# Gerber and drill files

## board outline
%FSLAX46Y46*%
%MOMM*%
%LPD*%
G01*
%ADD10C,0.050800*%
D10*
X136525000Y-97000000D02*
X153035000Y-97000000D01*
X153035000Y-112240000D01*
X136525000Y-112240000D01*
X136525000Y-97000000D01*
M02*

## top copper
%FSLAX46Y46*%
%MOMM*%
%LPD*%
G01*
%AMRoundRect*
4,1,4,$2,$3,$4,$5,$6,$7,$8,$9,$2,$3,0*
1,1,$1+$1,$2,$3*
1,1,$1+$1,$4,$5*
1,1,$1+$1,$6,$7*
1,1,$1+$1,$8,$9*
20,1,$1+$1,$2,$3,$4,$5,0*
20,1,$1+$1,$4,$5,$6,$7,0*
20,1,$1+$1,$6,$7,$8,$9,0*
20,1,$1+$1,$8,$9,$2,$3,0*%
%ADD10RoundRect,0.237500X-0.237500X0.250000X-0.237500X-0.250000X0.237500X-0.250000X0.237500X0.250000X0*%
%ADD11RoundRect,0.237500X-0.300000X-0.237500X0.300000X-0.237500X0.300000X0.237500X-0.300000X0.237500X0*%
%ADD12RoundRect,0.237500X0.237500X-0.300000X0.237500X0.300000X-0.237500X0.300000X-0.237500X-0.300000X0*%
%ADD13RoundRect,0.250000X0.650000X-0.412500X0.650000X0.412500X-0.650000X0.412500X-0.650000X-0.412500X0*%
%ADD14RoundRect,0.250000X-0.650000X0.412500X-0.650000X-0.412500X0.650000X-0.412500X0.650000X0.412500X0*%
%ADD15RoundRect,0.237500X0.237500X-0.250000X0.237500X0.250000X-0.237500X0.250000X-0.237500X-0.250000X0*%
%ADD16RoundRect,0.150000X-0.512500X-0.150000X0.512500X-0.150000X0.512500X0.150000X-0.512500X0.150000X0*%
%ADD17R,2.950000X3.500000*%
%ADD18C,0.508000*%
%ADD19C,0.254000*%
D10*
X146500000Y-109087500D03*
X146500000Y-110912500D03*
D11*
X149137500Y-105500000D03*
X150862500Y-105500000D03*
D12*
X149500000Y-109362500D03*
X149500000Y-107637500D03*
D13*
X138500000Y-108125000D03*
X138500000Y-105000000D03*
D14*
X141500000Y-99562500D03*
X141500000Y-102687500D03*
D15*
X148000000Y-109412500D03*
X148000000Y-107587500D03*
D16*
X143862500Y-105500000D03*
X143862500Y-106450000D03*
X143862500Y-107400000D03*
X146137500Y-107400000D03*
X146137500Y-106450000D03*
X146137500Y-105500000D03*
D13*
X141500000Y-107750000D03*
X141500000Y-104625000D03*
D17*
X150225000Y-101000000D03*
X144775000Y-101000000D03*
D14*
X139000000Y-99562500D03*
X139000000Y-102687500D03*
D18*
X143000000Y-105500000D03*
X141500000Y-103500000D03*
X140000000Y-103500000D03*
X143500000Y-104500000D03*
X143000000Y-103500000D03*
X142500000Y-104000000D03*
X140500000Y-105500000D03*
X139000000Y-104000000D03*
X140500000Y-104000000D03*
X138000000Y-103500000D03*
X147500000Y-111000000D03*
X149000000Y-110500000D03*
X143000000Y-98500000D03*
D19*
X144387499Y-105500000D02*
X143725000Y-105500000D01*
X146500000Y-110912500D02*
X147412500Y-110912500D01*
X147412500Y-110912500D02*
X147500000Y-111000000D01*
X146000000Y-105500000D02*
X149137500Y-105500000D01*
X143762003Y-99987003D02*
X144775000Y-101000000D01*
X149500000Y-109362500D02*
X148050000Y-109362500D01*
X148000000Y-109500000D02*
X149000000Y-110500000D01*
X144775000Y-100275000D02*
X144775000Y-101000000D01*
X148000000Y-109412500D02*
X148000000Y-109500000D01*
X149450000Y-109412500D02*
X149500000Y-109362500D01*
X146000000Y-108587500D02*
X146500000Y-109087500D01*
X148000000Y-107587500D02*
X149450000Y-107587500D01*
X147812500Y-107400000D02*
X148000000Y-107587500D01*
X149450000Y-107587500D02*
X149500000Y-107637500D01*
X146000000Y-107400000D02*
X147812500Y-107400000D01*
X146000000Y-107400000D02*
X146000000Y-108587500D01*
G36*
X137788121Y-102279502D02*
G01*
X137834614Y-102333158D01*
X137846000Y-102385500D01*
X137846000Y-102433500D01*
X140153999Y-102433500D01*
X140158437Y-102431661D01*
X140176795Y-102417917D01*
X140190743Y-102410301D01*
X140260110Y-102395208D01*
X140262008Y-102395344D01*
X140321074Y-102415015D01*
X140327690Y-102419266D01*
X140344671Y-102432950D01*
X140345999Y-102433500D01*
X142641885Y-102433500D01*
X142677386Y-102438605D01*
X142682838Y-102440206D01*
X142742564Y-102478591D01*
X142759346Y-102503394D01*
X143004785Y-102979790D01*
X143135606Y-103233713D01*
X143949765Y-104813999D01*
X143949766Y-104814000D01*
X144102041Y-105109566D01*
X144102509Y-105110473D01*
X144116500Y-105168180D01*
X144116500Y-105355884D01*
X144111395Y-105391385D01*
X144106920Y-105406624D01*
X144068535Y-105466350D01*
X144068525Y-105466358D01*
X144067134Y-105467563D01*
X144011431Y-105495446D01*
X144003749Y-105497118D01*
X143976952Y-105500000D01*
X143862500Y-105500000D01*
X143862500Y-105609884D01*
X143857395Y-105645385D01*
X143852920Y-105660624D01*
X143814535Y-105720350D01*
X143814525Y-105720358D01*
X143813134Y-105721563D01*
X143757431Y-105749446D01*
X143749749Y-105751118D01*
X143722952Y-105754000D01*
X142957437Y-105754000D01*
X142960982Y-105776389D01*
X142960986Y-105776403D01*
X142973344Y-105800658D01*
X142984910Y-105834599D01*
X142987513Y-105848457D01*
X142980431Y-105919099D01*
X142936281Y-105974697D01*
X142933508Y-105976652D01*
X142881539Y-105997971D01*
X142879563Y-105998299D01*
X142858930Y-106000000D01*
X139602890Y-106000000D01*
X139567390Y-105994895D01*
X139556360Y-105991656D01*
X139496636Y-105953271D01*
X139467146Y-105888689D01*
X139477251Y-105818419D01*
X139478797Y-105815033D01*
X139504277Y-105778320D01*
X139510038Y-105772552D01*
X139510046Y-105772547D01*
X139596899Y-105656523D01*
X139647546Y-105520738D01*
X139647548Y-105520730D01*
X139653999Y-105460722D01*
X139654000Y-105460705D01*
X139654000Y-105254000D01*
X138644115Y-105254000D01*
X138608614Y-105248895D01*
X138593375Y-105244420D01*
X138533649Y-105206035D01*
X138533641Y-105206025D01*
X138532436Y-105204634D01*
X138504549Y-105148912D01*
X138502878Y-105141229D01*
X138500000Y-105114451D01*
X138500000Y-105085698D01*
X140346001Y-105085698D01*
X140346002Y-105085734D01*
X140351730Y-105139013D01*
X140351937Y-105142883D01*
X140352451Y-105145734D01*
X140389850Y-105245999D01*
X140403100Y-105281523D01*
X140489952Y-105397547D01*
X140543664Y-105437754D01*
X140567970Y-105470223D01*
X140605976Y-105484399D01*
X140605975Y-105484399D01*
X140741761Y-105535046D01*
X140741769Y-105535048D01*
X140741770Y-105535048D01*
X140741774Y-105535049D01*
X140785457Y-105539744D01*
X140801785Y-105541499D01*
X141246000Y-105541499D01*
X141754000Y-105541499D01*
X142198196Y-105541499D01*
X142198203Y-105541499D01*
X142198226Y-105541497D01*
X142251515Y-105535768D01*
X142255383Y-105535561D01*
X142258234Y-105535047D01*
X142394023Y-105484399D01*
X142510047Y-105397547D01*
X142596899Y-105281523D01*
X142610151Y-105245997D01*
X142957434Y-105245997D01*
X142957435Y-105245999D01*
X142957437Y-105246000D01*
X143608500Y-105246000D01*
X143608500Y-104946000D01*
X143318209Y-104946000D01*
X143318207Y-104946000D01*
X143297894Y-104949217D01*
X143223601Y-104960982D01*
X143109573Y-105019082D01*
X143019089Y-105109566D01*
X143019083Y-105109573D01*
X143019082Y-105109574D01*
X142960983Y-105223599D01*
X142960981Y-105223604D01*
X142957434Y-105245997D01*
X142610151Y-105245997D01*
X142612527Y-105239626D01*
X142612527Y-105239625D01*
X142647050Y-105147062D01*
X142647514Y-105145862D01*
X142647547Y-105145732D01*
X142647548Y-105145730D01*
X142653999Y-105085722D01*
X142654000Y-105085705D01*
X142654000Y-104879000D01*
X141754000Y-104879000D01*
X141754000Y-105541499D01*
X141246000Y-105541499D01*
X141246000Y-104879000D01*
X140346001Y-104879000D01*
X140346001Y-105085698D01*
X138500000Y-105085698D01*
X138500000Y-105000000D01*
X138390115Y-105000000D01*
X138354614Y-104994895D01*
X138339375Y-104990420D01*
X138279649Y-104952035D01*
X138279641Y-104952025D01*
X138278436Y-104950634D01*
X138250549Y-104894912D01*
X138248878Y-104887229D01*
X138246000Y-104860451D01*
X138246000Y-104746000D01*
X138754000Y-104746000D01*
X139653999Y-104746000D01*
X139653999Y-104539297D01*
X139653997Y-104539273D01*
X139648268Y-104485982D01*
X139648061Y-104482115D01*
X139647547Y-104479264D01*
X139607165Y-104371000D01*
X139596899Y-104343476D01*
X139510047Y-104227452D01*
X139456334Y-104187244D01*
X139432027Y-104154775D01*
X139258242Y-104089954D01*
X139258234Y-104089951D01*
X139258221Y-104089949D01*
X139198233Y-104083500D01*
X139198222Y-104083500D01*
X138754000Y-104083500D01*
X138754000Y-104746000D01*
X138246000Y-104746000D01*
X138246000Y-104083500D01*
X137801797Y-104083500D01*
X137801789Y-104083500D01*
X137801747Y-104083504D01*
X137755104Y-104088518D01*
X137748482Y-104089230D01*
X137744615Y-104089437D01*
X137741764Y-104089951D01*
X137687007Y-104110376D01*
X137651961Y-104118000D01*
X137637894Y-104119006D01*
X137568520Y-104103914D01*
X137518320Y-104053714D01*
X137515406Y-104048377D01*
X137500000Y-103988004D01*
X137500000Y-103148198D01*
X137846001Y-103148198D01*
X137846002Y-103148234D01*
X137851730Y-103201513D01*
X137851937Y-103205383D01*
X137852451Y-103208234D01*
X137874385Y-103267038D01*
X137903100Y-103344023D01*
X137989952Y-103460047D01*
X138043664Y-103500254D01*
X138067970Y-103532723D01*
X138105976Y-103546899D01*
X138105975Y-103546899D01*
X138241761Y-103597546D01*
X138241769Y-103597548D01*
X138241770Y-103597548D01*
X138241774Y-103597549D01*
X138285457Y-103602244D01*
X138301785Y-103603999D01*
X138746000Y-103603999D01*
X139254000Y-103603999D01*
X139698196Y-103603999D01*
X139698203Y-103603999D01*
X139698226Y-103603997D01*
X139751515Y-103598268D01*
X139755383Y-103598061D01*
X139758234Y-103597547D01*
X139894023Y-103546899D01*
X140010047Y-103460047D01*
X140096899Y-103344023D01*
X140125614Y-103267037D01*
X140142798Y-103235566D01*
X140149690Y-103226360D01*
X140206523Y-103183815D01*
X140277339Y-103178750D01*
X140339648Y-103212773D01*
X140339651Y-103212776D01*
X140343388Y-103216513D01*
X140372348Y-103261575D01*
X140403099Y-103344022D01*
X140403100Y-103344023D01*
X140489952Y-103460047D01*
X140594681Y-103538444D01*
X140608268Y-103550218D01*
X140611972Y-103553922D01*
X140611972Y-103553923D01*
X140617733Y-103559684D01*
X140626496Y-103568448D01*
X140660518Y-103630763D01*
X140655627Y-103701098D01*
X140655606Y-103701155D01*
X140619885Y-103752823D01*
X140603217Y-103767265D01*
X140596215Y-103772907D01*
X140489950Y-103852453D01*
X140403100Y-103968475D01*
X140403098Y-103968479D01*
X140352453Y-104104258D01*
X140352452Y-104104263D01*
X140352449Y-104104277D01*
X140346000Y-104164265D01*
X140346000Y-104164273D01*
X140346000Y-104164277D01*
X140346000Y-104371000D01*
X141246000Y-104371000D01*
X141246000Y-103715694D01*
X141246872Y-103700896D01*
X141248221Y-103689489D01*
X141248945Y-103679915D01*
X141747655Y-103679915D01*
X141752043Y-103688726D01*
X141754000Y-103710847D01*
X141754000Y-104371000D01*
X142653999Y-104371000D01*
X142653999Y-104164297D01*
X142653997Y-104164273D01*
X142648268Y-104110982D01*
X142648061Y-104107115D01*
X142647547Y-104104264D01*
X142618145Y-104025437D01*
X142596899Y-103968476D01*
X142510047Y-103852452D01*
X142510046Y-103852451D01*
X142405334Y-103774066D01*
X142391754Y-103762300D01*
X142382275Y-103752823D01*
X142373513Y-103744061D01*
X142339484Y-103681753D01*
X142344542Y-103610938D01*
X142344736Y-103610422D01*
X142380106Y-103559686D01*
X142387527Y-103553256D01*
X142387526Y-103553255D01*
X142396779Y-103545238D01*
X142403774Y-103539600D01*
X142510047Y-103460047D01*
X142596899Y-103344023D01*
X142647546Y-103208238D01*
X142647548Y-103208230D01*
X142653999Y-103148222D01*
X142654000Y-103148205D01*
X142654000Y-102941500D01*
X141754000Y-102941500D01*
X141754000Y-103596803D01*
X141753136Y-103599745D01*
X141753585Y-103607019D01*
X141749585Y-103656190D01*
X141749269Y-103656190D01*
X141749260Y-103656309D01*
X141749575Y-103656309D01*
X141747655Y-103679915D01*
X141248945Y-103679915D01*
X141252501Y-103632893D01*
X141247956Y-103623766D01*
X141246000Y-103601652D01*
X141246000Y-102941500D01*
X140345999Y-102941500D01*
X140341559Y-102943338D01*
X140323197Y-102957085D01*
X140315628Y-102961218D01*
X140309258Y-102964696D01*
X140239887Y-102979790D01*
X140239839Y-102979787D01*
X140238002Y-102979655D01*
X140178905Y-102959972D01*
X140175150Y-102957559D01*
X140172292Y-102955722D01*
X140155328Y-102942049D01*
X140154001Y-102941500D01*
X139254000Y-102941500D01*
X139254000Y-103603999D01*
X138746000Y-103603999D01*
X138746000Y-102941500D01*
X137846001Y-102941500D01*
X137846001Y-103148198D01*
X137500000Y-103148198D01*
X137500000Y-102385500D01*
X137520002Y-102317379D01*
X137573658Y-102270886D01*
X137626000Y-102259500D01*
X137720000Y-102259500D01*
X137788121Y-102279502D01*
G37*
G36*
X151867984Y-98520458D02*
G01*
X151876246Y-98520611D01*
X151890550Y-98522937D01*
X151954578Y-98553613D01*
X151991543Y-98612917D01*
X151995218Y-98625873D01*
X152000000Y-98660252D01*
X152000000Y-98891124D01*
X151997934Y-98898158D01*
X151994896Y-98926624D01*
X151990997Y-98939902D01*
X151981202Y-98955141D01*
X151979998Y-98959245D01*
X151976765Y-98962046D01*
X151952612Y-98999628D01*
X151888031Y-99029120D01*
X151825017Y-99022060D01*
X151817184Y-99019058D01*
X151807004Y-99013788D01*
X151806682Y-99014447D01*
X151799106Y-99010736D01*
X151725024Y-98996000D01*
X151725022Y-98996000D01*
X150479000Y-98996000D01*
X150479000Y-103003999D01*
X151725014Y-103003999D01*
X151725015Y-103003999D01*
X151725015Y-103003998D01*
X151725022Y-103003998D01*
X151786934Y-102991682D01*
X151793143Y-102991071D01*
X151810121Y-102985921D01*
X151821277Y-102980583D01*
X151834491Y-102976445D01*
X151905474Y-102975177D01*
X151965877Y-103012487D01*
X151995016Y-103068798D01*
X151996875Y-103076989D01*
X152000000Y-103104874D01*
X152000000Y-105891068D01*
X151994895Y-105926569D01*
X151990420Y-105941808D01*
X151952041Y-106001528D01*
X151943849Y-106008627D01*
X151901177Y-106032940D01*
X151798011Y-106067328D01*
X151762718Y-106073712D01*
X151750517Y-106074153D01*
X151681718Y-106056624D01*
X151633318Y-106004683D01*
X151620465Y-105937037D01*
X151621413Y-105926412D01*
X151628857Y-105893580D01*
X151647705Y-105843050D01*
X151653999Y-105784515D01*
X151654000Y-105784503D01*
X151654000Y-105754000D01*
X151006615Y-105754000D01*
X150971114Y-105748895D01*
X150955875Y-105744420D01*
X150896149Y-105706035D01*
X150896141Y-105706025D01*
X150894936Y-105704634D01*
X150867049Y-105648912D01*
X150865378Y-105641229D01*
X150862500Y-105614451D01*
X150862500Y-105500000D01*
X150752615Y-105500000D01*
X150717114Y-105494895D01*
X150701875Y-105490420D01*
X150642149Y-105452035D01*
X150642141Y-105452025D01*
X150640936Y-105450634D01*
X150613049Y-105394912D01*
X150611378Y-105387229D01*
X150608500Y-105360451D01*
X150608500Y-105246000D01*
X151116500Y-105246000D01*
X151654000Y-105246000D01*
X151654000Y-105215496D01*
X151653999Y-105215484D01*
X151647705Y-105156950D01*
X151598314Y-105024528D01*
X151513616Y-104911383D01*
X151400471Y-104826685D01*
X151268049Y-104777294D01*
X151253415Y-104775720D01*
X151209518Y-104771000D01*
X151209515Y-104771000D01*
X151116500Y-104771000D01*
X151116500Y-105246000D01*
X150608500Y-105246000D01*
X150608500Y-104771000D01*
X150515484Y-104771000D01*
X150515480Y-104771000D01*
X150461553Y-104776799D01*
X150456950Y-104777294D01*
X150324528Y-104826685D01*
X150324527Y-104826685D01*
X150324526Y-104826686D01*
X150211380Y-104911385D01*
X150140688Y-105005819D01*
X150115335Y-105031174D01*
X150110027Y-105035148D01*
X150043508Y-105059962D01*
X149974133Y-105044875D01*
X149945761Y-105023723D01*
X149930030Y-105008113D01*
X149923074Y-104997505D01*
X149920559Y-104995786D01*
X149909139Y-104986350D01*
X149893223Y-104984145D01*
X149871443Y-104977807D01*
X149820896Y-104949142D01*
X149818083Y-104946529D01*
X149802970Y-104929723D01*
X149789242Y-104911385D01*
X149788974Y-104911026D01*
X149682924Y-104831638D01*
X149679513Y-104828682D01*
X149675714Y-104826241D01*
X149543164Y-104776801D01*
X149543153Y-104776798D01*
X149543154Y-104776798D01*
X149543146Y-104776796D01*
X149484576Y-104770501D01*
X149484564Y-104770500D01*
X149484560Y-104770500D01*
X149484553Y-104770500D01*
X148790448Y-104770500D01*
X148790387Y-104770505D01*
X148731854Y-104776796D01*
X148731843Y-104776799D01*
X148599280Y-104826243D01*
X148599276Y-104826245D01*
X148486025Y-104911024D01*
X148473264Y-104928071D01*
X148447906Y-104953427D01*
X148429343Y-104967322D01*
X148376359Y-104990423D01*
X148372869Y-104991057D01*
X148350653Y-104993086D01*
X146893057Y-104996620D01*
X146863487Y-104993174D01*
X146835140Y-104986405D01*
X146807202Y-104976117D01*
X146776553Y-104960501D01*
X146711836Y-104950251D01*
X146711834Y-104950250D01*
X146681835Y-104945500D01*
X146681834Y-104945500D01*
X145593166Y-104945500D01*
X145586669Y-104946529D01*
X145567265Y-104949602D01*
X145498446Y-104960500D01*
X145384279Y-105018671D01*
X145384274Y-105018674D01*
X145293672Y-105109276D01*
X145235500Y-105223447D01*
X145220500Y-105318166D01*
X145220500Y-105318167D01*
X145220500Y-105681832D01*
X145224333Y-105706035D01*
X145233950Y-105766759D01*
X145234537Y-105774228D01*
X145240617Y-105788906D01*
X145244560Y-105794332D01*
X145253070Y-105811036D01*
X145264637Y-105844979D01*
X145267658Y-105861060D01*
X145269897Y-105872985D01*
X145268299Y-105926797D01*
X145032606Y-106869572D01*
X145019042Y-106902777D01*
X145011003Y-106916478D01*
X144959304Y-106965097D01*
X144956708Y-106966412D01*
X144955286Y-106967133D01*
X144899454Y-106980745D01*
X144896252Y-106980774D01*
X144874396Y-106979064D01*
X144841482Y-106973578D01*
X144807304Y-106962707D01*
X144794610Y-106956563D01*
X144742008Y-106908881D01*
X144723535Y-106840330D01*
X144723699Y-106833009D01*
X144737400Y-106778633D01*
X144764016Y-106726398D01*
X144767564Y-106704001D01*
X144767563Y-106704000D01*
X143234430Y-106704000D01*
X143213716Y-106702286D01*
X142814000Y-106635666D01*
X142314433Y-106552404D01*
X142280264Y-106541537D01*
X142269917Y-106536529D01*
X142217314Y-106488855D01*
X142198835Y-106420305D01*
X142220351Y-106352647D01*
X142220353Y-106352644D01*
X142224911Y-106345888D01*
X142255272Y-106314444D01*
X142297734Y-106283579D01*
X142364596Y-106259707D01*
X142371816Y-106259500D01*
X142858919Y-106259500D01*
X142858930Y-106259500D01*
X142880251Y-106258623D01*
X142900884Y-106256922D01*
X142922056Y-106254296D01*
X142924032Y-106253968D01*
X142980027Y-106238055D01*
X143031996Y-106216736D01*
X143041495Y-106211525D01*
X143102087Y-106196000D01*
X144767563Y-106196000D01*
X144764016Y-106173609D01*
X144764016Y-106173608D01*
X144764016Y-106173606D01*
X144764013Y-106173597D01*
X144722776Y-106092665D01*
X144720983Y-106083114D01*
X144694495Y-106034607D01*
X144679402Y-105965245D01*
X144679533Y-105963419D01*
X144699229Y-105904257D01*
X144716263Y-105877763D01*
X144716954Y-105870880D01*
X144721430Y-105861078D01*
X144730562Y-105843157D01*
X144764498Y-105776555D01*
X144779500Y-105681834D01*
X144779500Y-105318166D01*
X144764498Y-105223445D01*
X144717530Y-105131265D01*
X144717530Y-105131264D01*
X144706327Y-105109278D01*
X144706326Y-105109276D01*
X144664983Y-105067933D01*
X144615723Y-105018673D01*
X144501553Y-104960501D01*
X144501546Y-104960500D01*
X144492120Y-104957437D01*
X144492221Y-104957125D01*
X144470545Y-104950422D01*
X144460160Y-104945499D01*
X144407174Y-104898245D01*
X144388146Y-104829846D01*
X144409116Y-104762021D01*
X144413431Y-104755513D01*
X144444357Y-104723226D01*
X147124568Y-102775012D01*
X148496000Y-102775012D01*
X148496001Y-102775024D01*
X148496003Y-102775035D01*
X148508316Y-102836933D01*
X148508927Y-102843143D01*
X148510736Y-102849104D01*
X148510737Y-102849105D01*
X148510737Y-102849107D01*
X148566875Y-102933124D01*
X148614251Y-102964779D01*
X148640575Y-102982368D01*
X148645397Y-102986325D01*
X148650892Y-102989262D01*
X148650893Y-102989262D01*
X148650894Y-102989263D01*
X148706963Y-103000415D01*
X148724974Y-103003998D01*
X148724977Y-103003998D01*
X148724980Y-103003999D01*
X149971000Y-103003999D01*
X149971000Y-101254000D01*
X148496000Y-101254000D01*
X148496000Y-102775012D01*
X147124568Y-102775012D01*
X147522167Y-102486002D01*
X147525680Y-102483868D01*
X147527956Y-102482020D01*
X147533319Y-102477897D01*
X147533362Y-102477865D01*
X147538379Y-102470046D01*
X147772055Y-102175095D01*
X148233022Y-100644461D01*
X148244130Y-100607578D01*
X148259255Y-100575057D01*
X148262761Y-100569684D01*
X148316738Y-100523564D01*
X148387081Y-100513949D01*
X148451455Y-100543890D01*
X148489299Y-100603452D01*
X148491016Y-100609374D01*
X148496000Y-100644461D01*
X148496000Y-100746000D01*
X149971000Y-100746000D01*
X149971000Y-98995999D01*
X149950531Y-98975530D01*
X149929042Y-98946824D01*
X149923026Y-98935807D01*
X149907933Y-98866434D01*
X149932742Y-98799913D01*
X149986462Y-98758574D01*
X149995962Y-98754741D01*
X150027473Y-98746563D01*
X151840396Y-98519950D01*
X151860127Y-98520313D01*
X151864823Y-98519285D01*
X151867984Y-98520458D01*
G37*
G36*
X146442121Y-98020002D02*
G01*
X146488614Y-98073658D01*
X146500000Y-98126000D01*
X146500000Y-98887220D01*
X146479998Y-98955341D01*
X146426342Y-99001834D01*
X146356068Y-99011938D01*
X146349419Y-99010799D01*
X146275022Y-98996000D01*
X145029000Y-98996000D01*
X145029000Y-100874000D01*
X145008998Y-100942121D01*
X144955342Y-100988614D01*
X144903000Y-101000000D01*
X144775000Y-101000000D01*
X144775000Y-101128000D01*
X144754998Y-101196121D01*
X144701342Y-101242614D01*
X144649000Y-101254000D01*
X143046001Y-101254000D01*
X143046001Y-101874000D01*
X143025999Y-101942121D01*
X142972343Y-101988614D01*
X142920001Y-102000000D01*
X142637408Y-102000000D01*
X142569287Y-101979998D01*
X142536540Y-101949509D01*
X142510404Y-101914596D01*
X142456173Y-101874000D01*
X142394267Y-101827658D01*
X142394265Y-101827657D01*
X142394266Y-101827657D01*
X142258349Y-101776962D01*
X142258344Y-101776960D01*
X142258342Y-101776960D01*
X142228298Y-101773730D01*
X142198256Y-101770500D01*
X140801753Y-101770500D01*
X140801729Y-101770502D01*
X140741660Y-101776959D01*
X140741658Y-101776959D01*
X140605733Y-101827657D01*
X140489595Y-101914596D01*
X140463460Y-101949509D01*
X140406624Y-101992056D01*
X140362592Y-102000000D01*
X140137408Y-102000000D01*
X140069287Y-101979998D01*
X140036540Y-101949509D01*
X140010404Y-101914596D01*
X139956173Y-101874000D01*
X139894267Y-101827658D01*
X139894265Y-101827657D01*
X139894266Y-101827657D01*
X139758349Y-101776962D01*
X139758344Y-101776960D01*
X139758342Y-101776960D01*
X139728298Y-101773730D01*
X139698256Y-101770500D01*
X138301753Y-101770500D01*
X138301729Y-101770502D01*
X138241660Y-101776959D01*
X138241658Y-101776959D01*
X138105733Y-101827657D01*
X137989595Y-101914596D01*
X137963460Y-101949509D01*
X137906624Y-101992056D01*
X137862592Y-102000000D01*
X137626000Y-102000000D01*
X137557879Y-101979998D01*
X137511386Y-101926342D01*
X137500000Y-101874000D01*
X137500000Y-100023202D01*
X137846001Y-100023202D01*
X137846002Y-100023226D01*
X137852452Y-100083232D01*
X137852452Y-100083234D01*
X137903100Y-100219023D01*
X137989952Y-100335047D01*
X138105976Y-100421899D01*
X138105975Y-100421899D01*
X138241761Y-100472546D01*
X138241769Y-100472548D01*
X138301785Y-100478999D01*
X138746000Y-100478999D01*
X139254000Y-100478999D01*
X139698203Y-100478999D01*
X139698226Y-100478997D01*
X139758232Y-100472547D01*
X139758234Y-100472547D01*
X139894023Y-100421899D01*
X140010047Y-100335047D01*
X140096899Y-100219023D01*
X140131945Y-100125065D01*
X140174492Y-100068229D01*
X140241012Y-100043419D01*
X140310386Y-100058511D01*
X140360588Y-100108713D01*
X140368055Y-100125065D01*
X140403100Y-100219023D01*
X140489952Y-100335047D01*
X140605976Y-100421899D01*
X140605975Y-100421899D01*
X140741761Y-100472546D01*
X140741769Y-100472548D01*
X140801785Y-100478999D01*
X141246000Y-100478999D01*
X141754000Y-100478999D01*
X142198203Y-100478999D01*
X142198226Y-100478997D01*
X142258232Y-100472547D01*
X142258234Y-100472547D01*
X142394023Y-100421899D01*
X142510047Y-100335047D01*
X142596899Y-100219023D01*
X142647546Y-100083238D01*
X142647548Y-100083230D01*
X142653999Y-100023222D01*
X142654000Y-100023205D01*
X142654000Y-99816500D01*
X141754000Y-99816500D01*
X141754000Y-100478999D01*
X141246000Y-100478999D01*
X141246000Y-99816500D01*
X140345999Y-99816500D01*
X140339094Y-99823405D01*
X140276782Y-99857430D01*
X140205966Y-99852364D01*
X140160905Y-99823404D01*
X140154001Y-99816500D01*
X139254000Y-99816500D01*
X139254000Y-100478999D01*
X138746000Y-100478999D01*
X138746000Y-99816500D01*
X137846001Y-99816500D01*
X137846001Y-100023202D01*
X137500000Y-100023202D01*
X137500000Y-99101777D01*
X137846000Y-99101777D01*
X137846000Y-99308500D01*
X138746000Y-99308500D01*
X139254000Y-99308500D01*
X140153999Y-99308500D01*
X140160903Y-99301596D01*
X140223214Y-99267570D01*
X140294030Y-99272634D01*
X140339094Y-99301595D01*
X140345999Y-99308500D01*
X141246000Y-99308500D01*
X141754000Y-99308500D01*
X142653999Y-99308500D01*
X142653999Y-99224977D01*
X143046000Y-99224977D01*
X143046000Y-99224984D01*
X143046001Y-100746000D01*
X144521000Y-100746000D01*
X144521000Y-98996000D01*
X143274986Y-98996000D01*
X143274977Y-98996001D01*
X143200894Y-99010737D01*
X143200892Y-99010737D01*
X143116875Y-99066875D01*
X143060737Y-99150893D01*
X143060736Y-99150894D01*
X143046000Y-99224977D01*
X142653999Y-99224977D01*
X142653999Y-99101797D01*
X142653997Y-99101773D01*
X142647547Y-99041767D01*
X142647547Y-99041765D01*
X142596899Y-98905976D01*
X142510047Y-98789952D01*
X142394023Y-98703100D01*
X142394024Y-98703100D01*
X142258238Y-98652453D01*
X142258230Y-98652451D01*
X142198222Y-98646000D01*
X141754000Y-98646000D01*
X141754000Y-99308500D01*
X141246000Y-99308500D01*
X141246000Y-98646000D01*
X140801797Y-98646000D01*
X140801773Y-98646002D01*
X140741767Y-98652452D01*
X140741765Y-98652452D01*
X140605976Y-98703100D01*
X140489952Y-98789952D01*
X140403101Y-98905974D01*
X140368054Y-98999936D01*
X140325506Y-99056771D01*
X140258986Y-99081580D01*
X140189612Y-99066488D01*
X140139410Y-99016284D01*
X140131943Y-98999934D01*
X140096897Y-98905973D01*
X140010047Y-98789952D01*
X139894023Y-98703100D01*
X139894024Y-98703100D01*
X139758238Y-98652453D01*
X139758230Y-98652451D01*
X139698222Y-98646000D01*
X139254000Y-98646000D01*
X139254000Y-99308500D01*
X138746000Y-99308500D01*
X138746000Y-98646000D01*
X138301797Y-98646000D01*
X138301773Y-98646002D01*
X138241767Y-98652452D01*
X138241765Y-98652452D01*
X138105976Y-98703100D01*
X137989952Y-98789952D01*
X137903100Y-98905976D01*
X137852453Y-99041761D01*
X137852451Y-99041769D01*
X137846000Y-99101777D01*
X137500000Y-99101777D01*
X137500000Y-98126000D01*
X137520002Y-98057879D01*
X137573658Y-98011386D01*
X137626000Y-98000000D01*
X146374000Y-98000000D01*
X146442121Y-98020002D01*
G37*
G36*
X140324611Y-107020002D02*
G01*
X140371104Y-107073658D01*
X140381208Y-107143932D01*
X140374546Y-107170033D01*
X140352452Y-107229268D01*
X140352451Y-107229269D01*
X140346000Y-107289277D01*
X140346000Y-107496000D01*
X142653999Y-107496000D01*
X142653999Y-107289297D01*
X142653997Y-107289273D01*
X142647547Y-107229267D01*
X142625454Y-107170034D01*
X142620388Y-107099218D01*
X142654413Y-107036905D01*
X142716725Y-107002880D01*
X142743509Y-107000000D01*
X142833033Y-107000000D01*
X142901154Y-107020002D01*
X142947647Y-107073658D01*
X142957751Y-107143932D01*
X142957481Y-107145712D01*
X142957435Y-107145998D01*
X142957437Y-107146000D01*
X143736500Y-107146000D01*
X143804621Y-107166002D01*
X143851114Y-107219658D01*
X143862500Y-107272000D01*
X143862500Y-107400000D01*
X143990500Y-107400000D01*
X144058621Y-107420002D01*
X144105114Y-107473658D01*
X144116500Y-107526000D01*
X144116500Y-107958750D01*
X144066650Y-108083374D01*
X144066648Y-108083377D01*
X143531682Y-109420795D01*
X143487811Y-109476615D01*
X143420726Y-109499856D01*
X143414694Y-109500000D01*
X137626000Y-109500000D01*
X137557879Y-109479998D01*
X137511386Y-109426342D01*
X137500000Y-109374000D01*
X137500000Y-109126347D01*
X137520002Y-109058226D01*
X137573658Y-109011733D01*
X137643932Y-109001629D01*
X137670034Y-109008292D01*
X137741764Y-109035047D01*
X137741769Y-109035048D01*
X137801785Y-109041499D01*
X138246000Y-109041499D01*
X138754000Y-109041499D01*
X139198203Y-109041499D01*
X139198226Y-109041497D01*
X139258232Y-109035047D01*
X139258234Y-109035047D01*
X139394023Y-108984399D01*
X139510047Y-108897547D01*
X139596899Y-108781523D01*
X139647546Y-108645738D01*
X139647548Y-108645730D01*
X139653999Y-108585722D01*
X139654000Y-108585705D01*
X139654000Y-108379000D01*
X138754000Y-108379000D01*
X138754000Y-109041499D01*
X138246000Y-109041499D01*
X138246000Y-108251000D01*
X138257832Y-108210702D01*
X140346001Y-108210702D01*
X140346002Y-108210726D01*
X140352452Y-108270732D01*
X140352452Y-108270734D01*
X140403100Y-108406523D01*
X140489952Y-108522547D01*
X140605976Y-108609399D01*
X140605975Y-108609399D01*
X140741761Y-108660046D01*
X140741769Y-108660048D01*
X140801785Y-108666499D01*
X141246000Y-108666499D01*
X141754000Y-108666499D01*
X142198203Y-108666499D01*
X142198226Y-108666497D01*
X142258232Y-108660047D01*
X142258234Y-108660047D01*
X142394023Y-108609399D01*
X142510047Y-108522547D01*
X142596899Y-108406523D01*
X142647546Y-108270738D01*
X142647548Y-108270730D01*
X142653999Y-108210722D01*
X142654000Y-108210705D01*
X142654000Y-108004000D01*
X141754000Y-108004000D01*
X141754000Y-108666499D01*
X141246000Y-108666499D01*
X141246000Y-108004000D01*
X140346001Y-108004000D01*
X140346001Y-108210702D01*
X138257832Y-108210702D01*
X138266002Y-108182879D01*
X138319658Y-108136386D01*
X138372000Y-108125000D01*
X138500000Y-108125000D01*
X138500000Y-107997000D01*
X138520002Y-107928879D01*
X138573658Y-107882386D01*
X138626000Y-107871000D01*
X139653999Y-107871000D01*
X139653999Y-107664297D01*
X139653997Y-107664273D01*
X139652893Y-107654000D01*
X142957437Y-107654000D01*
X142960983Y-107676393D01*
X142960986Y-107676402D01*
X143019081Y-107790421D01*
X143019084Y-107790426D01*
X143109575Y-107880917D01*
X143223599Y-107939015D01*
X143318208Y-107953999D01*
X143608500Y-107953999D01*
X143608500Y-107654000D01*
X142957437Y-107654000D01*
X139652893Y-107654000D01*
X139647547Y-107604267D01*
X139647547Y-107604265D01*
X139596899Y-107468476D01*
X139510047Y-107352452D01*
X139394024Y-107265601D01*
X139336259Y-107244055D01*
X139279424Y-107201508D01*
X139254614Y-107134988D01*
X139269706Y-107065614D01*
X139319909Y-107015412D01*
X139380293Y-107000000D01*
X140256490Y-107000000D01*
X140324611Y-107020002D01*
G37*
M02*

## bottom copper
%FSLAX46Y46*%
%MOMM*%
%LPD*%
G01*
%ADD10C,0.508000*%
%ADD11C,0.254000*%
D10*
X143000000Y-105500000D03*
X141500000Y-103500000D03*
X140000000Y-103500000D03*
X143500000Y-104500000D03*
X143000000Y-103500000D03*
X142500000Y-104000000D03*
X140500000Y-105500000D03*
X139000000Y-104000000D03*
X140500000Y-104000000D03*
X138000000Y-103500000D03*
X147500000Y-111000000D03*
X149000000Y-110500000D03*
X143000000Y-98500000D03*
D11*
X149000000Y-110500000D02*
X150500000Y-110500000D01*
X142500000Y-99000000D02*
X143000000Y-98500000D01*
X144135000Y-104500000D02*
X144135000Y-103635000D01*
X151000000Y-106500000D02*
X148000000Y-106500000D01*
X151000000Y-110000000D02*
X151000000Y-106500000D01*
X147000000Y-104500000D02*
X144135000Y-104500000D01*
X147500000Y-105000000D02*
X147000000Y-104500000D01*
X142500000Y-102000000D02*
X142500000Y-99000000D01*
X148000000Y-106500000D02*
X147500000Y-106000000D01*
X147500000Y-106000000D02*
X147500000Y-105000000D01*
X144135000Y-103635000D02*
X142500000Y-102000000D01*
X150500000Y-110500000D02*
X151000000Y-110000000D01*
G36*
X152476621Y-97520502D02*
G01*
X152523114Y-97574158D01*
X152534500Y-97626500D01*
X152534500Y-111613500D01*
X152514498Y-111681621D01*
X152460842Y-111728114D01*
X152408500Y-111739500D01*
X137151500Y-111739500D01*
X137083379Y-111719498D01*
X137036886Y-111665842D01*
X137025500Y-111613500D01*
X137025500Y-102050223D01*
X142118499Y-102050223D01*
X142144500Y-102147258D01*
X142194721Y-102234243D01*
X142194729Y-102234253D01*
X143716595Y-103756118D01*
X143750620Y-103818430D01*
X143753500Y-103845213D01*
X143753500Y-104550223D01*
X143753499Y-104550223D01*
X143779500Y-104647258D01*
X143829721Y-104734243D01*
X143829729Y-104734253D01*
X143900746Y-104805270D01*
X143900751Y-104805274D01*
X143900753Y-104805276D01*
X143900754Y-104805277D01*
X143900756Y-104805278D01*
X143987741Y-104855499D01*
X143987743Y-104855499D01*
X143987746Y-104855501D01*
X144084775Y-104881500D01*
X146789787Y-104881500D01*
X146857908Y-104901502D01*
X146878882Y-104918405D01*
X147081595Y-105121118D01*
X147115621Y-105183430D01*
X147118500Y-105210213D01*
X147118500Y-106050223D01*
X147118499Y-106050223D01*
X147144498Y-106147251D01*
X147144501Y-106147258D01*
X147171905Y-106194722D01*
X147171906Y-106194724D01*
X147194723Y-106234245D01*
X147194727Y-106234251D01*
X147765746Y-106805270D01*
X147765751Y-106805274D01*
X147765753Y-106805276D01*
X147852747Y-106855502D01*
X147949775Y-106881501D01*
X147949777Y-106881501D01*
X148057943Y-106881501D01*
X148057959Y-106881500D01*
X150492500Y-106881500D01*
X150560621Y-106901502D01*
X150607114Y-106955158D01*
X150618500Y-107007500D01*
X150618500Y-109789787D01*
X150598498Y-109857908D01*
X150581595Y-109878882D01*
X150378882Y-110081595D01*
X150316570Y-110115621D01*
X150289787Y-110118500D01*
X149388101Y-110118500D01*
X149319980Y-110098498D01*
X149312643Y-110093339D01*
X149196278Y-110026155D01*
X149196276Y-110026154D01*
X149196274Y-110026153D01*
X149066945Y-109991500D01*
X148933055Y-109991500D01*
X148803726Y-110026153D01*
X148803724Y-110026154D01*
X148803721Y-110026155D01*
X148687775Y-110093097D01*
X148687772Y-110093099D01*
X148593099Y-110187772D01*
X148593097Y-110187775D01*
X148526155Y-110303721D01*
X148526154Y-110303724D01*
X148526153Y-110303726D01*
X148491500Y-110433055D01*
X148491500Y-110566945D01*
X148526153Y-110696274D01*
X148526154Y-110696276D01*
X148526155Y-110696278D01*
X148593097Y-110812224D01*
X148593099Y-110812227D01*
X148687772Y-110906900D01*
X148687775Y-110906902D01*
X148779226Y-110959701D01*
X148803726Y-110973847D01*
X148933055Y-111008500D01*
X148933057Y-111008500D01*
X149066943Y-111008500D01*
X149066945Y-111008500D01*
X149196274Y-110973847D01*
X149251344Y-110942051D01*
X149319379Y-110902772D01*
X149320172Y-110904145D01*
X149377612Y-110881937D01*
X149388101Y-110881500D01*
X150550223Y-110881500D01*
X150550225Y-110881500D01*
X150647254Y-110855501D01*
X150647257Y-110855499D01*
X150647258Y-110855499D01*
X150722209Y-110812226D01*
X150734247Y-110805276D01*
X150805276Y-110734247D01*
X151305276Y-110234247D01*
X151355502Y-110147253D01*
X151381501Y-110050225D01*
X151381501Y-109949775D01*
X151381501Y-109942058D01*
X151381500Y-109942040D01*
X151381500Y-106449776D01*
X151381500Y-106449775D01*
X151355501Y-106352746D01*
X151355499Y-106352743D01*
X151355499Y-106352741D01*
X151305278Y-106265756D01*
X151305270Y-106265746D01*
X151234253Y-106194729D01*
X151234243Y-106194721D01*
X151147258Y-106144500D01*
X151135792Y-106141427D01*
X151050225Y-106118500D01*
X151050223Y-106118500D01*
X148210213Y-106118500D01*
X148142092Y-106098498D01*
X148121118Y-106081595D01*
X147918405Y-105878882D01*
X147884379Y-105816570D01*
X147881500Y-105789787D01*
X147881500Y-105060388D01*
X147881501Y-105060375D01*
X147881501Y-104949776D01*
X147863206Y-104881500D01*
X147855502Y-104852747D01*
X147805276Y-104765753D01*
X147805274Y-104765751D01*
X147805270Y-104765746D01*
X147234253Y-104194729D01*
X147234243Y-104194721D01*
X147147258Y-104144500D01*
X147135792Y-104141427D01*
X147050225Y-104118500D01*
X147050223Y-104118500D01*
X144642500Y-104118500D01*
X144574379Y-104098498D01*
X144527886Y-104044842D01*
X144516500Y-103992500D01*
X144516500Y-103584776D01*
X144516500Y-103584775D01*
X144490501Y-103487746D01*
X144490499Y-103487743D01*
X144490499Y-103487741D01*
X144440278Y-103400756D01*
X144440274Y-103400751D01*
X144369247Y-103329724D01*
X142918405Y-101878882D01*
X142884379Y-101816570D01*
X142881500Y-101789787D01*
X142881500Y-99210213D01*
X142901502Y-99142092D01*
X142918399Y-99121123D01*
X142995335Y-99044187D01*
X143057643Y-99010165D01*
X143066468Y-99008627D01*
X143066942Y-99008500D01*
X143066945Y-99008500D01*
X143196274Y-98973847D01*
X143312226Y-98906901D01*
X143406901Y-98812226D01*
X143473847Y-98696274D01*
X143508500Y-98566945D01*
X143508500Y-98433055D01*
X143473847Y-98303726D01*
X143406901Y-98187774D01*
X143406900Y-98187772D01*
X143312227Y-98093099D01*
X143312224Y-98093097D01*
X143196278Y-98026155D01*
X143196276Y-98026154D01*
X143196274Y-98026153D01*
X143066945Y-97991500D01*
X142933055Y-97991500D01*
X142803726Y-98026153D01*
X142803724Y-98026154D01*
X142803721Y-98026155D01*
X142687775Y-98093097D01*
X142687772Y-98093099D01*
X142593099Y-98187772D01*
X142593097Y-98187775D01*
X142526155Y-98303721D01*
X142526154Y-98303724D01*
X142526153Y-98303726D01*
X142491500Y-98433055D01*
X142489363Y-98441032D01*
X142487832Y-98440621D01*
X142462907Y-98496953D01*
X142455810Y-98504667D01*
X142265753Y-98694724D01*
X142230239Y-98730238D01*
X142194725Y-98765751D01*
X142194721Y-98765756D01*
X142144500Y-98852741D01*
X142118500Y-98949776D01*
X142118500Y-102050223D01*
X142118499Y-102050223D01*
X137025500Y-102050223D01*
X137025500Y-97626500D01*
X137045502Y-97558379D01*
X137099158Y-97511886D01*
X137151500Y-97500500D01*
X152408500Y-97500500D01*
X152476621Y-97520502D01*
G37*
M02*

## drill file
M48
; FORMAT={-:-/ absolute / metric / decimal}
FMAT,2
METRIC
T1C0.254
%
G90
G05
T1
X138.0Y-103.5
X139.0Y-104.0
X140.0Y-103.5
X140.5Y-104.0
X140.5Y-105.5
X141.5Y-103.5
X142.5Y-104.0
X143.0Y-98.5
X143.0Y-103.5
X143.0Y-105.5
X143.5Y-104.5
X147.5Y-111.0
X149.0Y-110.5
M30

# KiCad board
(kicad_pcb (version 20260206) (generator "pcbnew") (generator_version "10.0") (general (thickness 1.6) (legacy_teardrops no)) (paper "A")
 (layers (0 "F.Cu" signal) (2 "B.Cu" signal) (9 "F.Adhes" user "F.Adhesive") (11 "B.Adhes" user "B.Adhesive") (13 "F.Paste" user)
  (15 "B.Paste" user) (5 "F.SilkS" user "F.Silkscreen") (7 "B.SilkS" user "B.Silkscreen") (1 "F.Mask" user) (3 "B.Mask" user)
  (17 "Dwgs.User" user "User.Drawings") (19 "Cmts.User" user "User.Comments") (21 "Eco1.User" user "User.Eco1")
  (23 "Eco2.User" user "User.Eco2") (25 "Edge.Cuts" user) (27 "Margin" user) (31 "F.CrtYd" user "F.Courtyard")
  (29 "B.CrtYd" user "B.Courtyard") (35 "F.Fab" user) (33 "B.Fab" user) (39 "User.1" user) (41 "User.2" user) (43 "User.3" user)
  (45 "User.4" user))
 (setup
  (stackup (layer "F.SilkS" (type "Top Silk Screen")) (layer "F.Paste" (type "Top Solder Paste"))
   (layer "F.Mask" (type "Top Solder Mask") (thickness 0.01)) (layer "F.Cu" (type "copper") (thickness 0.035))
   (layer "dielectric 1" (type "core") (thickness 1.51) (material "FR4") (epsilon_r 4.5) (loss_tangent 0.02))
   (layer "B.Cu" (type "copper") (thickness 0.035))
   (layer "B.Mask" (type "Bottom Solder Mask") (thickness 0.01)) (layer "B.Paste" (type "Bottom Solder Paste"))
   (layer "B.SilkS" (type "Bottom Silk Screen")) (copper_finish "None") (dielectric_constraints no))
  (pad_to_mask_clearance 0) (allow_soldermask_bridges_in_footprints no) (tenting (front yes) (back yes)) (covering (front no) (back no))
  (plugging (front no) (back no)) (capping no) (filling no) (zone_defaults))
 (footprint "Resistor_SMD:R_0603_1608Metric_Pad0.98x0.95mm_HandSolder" (layer "F.Cu") (at 146.5 110 -90)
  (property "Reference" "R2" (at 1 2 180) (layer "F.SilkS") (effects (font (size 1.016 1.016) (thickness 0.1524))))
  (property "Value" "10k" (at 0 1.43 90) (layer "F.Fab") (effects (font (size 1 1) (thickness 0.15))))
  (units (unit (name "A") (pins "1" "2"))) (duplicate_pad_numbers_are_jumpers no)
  (pad "1" smd roundrect (at -0.9125 0 270) (size 0.975 0.95) (layers "F.Cu" "F.Mask" "F.Paste") (roundrect_rratio 0.25) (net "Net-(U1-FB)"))
  (pad "2" smd roundrect (at 0.9125 0 270) (size 0.975 0.95) (layers "F.Cu" "F.Mask" "F.Paste") (roundrect_rratio 0.25) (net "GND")))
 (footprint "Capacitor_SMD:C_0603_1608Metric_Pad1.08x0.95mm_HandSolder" (layer "F.Cu") (at 150 105.5)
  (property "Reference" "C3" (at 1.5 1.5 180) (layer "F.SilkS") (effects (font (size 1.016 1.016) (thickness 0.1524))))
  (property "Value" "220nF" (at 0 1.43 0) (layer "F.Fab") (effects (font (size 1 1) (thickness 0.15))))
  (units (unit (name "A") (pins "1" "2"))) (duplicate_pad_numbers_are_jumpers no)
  (pad "1" smd roundrect (at -0.8625 0) (size 1.075 0.95) (layers "F.Cu" "F.Mask" "F.Paste") (roundrect_rratio 0.25) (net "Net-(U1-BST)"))
  (pad "2" smd roundrect (at 0.8625 0) (size 1.075 0.95) (layers "F.Cu" "F.Mask" "F.Paste") (roundrect_rratio 0.25) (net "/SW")))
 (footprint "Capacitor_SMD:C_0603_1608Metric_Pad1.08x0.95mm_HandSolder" (layer "F.Cu") (at 149.5 108.5 90)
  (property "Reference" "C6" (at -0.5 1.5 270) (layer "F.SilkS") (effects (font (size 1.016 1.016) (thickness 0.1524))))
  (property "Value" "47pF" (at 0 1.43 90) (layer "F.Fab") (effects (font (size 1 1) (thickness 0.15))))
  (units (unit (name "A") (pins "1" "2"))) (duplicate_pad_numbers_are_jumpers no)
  (pad "1" smd roundrect (at -0.8625 0 90) (size 1.075 0.95) (layers "F.Cu" "F.Mask" "F.Paste") (roundrect_rratio 0.25) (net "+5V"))
  (pad "2" smd roundrect (at 0.8625 0 90) (size 1.075 0.95) (layers "F.Cu" "F.Mask" "F.Paste") (roundrect_rratio 0.25) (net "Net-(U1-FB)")))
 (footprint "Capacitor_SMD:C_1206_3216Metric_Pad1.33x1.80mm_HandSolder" (layer "F.Cu") (at 138.5 106.5625 90)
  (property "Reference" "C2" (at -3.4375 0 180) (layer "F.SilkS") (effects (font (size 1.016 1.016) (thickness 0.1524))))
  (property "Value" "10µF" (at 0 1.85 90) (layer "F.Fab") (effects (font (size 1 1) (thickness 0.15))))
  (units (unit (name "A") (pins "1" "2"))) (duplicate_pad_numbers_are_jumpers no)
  (pad "1" smd roundrect (at -1.5625 0 90) (size 1.325 1.8) (layers "F.Cu" "F.Mask" "F.Paste") (roundrect_rratio 0.188679) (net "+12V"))
  (pad "2" smd roundrect (at 1.5625 0 90) (size 1.325 1.8) (layers "F.Cu" "F.Mask" "F.Paste") (roundrect_rratio 0.188679) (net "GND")))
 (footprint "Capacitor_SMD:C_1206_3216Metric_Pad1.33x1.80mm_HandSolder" (layer "F.Cu") (at 141.5 101.125 -90)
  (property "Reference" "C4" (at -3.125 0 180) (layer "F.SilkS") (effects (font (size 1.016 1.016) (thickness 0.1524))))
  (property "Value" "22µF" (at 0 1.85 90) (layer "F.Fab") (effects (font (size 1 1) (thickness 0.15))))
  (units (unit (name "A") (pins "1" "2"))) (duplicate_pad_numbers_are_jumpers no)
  (pad "1" smd roundrect (at -1.5625 0 270) (size 1.325 1.8) (layers "F.Cu" "F.Mask" "F.Paste") (roundrect_rratio 0.188679) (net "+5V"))
  (pad "2" smd roundrect (at 1.5625 0 270) (size 1.325 1.8) (layers "F.Cu" "F.Mask" "F.Paste") (roundrect_rratio 0.188679) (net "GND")))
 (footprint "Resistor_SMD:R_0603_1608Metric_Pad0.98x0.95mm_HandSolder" (layer "F.Cu") (at 148 108.5 90)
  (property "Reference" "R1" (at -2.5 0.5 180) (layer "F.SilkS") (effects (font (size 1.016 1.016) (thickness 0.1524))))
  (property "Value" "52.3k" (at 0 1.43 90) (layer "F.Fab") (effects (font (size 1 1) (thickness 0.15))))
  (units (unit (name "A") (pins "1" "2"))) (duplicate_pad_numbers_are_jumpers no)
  (pad "1" smd roundrect (at -0.9125 0 90) (size 0.975 0.95) (layers "F.Cu" "F.Mask" "F.Paste") (roundrect_rratio 0.25) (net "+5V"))
  (pad "2" smd roundrect (at 0.9125 0 90) (size 0.975 0.95) (layers "F.Cu" "F.Mask" "F.Paste") (roundrect_rratio 0.25) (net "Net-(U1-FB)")))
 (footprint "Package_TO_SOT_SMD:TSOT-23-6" (layer "F.Cu") (at 145 106.45)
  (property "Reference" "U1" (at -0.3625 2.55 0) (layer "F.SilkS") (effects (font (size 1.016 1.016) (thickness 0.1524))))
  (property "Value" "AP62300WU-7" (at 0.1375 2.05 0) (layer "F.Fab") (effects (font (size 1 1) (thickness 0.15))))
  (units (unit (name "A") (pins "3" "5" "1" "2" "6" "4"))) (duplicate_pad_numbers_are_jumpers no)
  (pad "1" smd roundrect (at -1.1375 -0.95) (size 1.325 0.6) (layers "F.Cu" "F.Mask" "F.Paste") (roundrect_rratio 0.25) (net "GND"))
  (pad "2" smd roundrect (at -1.1375 0) (size 1.325 0.6) (layers "F.Cu" "F.Mask" "F.Paste") (roundrect_rratio 0.25) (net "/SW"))
  (pad "3" smd roundrect (at -1.1375 0.95) (size 1.325 0.6) (layers "F.Cu" "F.Mask" "F.Paste") (roundrect_rratio 0.25) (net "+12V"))
  (pad "4" smd roundrect (at 1.1375 0.95) (size 1.325 0.6) (layers "F.Cu" "F.Mask" "F.Paste") (roundrect_rratio 0.25) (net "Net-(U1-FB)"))
  (pad "5" smd roundrect (at 1.1375 0) (size 1.325 0.6) (layers "F.Cu" "F.Mask" "F.Paste") (roundrect_rratio 0.25)
   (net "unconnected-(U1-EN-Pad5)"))
  (pad "6" smd roundrect (at 1.1375 -0.95) (size 1.325 0.6) (layers "F.Cu" "F.Mask" "F.Paste") (roundrect_rratio 0.25) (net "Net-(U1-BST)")))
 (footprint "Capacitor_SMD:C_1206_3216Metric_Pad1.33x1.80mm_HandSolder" (layer "F.Cu") (at 141.5 106.1875 90)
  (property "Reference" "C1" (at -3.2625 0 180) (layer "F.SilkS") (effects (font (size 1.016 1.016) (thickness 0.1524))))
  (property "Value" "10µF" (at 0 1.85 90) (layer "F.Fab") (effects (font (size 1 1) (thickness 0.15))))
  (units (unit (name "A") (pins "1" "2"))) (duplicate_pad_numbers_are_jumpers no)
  (pad "1" smd roundrect (at -1.5625 0 90) (size 1.325 1.8) (layers "F.Cu" "F.Mask" "F.Paste") (roundrect_rratio 0.188679) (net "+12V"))
  (pad "2" smd roundrect (at 1.5625 0 90) (size 1.325 1.8) (layers "F.Cu" "F.Mask" "F.Paste") (roundrect_rratio 0.188679) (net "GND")))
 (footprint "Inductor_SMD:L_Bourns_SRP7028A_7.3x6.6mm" (layer "F.Cu") (at 147.5 101 180)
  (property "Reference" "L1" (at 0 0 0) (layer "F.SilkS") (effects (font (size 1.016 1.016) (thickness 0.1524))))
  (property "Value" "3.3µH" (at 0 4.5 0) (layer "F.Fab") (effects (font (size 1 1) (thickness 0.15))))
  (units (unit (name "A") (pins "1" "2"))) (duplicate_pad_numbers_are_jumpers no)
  (pad "1" smd rect (at -2.725 0 180) (size 2.95 3.5) (layers "F.Cu" "F.Mask" "F.Paste") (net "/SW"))
  (pad "2" smd rect (at 2.725 0 180) (size 2.95 3.5) (layers "F.Cu" "F.Mask" "F.Paste") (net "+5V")))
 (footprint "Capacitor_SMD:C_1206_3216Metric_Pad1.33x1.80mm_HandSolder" (layer "F.Cu") (at 139 101.125 -90)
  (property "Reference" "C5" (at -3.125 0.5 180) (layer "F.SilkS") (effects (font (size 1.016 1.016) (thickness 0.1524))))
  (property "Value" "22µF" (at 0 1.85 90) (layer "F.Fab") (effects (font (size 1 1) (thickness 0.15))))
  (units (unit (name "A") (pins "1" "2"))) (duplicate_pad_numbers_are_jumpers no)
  (pad "1" smd roundrect (at -1.5625 0 270) (size 1.325 1.8) (layers "F.Cu" "F.Mask" "F.Paste") (roundrect_rratio 0.188679) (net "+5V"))
  (pad "2" smd roundrect (at 1.5625 0 270) (size 1.325 1.8) (layers "F.Cu" "F.Mask" "F.Paste") (roundrect_rratio 0.188679) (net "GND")))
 (gr_rect (start 136.525 97) (end 153.035 112.24) (stroke (width 0.0508) (type solid)) (fill no) (layer "Edge.Cuts"))
 (segment (start 144.387499 105.5) (end 143.725 105.5) (width 0.254) (layer "F.Cu") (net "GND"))
 (segment (start 146.5 110.9125) (end 147.4125 110.9125) (width 0.254) (layer "F.Cu") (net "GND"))
 (segment (start 147.4125 110.9125) (end 147.5 111) (width 0.254) (layer "F.Cu") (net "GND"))
 (via (at 143 105.5) (size 0.508) (drill 0.254) (layers "F.Cu" "B.Cu") (free yes) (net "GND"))
 (via (at 141.5 103.5) (size 0.508) (drill 0.254) (layers "F.Cu" "B.Cu") (free yes) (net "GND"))
 (via (at 140 103.5) (size 0.508) (drill 0.254) (layers "F.Cu" "B.Cu") (free yes) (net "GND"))
 (via (at 143.5 104.5) (size 0.508) (drill 0.254) (layers "F.Cu" "B.Cu") (free yes) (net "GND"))
 (via (at 143 103.5) (size 0.508) (drill 0.254) (layers "F.Cu" "B.Cu") (free yes) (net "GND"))
 (via (at 142.5 104) (size 0.508) (drill 0.254) (layers "F.Cu" "B.Cu") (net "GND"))
 (via (at 140.5 105.5) (size 0.508) (drill 0.254) (layers "F.Cu" "B.Cu") (free yes) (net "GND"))
 (via (at 139 104) (size 0.508) (drill 0.254) (layers "F.Cu" "B.Cu") (free yes) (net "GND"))
 (via (at 140.5 104) (size 0.508) (drill 0.254) (layers "F.Cu" "B.Cu") (free yes) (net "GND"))
 (via (at 138 103.5) (size 0.508) (drill 0.254) (layers "F.Cu" "B.Cu") (free yes) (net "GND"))
 (via (at 147.5 111) (size 0.508) (drill 0.254) (layers "F.Cu" "B.Cu") (free yes) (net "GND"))
 (segment (start 146 105.5) (end 149.1375 105.5) (width 0.254) (layer "F.Cu") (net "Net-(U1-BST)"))
 (segment (start 143.762003 99.987003) (end 144.775 101) (width 0.254) (layer "F.Cu") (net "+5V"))
 (segment (start 149.5 109.3625) (end 148.05 109.3625) (width 0.254) (layer "F.Cu") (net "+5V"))
 (segment (start 148 109.5) (end 149 110.5) (width 0.254) (layer "F.Cu") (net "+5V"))
 (segment (start 144.775 100.275) (end 144.775 101) (width 0.254) (layer "F.Cu") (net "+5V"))
 (segment (start 148 109.4125) (end 148 109.5) (width 0.254) (layer "F.Cu") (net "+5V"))
 (segment (start 149.45 109.4125) (end 149.5 109.3625) (width 0.254) (layer "F.Cu") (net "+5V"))
 (via (at 149 110.5) (size 0.508) (drill 0.254) (layers "F.Cu" "B.Cu") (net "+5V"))
 (via (at 143 98.5) (size 0.508) (drill 0.254) (layers "F.Cu" "B.Cu") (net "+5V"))
 (segment (start 149 110.5) (end 150.5 110.5) (width 0.254) (layer "B.Cu") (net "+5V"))
 (segment (start 142.5 99) (end 143 98.5) (width 0.254) (layer "B.Cu") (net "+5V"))
 (segment (start 144.135 104.5) (end 144.135 103.635) (width 0.254) (layer "B.Cu") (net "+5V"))
 (segment (start 151 106.5) (end 148 106.5) (width 0.254) (layer "B.Cu") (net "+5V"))
 (segment (start 151 110) (end 151 106.5) (width 0.254) (layer "B.Cu") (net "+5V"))
 (segment (start 147 104.5) (end 144.135 104.5) (width 0.254) (layer "B.Cu") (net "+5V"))
 (segment (start 147.5 105) (end 147 104.5) (width 0.254) (layer "B.Cu") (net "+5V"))
 (segment (start 142.5 102) (end 142.5 99) (width 0.254) (layer "B.Cu") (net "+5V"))
 (segment (start 148 106.5) (end 147.5 106) (width 0.254) (layer "B.Cu") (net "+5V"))
 (segment (start 147.5 106) (end 147.5 105) (width 0.254) (layer "B.Cu") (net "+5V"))
 (segment (start 144.135 103.635) (end 142.5 102) (width 0.254) (layer "B.Cu") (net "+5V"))
 (segment (start 150.5 110.5) (end 151 110) (width 0.254) (layer "B.Cu") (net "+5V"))
 (segment (start 146 108.5875) (end 146.5 109.0875) (width 0.254) (layer "F.Cu") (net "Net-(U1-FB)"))
 (segment (start 148 107.5875) (end 149.45 107.5875) (width 0.254) (layer "F.Cu") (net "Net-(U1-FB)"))
 (segment (start 147.8125 107.4) (end 148 107.5875) (width 0.254) (layer "F.Cu") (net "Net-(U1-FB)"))
 (segment (start 149.45 107.5875) (end 149.5 107.6375) (width 0.254) (layer "F.Cu") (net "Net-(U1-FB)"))
 (segment (start 146 107.4) (end 147.8125 107.4) (width 0.254) (layer "F.Cu") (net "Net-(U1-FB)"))
 (segment (start 146 107.4) (end 146 108.5875) (width 0.254) (layer "F.Cu") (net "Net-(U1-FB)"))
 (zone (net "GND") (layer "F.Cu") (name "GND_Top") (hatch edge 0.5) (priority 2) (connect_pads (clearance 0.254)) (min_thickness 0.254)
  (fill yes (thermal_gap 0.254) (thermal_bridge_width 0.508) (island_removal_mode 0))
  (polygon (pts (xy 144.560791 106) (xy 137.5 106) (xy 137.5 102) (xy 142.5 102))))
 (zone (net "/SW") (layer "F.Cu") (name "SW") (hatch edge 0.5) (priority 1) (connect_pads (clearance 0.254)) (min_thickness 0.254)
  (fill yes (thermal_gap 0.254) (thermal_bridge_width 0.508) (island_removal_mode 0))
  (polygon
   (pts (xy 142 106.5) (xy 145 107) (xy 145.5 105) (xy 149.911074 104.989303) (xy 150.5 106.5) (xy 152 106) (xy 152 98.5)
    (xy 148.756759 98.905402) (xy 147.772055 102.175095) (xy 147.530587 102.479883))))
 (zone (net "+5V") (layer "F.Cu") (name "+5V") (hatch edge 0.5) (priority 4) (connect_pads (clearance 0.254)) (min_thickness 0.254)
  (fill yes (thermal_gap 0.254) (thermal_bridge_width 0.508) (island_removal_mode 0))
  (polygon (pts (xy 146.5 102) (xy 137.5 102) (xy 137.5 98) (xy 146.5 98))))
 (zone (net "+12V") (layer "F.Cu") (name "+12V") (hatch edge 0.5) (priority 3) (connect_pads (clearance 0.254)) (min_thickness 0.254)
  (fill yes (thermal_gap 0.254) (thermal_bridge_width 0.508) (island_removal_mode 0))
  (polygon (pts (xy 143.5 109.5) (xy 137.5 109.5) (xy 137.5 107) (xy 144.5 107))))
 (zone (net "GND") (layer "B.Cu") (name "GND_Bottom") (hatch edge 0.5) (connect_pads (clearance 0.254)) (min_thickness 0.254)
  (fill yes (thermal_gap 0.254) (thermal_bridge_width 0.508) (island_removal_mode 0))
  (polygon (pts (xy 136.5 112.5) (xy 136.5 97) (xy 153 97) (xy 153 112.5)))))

